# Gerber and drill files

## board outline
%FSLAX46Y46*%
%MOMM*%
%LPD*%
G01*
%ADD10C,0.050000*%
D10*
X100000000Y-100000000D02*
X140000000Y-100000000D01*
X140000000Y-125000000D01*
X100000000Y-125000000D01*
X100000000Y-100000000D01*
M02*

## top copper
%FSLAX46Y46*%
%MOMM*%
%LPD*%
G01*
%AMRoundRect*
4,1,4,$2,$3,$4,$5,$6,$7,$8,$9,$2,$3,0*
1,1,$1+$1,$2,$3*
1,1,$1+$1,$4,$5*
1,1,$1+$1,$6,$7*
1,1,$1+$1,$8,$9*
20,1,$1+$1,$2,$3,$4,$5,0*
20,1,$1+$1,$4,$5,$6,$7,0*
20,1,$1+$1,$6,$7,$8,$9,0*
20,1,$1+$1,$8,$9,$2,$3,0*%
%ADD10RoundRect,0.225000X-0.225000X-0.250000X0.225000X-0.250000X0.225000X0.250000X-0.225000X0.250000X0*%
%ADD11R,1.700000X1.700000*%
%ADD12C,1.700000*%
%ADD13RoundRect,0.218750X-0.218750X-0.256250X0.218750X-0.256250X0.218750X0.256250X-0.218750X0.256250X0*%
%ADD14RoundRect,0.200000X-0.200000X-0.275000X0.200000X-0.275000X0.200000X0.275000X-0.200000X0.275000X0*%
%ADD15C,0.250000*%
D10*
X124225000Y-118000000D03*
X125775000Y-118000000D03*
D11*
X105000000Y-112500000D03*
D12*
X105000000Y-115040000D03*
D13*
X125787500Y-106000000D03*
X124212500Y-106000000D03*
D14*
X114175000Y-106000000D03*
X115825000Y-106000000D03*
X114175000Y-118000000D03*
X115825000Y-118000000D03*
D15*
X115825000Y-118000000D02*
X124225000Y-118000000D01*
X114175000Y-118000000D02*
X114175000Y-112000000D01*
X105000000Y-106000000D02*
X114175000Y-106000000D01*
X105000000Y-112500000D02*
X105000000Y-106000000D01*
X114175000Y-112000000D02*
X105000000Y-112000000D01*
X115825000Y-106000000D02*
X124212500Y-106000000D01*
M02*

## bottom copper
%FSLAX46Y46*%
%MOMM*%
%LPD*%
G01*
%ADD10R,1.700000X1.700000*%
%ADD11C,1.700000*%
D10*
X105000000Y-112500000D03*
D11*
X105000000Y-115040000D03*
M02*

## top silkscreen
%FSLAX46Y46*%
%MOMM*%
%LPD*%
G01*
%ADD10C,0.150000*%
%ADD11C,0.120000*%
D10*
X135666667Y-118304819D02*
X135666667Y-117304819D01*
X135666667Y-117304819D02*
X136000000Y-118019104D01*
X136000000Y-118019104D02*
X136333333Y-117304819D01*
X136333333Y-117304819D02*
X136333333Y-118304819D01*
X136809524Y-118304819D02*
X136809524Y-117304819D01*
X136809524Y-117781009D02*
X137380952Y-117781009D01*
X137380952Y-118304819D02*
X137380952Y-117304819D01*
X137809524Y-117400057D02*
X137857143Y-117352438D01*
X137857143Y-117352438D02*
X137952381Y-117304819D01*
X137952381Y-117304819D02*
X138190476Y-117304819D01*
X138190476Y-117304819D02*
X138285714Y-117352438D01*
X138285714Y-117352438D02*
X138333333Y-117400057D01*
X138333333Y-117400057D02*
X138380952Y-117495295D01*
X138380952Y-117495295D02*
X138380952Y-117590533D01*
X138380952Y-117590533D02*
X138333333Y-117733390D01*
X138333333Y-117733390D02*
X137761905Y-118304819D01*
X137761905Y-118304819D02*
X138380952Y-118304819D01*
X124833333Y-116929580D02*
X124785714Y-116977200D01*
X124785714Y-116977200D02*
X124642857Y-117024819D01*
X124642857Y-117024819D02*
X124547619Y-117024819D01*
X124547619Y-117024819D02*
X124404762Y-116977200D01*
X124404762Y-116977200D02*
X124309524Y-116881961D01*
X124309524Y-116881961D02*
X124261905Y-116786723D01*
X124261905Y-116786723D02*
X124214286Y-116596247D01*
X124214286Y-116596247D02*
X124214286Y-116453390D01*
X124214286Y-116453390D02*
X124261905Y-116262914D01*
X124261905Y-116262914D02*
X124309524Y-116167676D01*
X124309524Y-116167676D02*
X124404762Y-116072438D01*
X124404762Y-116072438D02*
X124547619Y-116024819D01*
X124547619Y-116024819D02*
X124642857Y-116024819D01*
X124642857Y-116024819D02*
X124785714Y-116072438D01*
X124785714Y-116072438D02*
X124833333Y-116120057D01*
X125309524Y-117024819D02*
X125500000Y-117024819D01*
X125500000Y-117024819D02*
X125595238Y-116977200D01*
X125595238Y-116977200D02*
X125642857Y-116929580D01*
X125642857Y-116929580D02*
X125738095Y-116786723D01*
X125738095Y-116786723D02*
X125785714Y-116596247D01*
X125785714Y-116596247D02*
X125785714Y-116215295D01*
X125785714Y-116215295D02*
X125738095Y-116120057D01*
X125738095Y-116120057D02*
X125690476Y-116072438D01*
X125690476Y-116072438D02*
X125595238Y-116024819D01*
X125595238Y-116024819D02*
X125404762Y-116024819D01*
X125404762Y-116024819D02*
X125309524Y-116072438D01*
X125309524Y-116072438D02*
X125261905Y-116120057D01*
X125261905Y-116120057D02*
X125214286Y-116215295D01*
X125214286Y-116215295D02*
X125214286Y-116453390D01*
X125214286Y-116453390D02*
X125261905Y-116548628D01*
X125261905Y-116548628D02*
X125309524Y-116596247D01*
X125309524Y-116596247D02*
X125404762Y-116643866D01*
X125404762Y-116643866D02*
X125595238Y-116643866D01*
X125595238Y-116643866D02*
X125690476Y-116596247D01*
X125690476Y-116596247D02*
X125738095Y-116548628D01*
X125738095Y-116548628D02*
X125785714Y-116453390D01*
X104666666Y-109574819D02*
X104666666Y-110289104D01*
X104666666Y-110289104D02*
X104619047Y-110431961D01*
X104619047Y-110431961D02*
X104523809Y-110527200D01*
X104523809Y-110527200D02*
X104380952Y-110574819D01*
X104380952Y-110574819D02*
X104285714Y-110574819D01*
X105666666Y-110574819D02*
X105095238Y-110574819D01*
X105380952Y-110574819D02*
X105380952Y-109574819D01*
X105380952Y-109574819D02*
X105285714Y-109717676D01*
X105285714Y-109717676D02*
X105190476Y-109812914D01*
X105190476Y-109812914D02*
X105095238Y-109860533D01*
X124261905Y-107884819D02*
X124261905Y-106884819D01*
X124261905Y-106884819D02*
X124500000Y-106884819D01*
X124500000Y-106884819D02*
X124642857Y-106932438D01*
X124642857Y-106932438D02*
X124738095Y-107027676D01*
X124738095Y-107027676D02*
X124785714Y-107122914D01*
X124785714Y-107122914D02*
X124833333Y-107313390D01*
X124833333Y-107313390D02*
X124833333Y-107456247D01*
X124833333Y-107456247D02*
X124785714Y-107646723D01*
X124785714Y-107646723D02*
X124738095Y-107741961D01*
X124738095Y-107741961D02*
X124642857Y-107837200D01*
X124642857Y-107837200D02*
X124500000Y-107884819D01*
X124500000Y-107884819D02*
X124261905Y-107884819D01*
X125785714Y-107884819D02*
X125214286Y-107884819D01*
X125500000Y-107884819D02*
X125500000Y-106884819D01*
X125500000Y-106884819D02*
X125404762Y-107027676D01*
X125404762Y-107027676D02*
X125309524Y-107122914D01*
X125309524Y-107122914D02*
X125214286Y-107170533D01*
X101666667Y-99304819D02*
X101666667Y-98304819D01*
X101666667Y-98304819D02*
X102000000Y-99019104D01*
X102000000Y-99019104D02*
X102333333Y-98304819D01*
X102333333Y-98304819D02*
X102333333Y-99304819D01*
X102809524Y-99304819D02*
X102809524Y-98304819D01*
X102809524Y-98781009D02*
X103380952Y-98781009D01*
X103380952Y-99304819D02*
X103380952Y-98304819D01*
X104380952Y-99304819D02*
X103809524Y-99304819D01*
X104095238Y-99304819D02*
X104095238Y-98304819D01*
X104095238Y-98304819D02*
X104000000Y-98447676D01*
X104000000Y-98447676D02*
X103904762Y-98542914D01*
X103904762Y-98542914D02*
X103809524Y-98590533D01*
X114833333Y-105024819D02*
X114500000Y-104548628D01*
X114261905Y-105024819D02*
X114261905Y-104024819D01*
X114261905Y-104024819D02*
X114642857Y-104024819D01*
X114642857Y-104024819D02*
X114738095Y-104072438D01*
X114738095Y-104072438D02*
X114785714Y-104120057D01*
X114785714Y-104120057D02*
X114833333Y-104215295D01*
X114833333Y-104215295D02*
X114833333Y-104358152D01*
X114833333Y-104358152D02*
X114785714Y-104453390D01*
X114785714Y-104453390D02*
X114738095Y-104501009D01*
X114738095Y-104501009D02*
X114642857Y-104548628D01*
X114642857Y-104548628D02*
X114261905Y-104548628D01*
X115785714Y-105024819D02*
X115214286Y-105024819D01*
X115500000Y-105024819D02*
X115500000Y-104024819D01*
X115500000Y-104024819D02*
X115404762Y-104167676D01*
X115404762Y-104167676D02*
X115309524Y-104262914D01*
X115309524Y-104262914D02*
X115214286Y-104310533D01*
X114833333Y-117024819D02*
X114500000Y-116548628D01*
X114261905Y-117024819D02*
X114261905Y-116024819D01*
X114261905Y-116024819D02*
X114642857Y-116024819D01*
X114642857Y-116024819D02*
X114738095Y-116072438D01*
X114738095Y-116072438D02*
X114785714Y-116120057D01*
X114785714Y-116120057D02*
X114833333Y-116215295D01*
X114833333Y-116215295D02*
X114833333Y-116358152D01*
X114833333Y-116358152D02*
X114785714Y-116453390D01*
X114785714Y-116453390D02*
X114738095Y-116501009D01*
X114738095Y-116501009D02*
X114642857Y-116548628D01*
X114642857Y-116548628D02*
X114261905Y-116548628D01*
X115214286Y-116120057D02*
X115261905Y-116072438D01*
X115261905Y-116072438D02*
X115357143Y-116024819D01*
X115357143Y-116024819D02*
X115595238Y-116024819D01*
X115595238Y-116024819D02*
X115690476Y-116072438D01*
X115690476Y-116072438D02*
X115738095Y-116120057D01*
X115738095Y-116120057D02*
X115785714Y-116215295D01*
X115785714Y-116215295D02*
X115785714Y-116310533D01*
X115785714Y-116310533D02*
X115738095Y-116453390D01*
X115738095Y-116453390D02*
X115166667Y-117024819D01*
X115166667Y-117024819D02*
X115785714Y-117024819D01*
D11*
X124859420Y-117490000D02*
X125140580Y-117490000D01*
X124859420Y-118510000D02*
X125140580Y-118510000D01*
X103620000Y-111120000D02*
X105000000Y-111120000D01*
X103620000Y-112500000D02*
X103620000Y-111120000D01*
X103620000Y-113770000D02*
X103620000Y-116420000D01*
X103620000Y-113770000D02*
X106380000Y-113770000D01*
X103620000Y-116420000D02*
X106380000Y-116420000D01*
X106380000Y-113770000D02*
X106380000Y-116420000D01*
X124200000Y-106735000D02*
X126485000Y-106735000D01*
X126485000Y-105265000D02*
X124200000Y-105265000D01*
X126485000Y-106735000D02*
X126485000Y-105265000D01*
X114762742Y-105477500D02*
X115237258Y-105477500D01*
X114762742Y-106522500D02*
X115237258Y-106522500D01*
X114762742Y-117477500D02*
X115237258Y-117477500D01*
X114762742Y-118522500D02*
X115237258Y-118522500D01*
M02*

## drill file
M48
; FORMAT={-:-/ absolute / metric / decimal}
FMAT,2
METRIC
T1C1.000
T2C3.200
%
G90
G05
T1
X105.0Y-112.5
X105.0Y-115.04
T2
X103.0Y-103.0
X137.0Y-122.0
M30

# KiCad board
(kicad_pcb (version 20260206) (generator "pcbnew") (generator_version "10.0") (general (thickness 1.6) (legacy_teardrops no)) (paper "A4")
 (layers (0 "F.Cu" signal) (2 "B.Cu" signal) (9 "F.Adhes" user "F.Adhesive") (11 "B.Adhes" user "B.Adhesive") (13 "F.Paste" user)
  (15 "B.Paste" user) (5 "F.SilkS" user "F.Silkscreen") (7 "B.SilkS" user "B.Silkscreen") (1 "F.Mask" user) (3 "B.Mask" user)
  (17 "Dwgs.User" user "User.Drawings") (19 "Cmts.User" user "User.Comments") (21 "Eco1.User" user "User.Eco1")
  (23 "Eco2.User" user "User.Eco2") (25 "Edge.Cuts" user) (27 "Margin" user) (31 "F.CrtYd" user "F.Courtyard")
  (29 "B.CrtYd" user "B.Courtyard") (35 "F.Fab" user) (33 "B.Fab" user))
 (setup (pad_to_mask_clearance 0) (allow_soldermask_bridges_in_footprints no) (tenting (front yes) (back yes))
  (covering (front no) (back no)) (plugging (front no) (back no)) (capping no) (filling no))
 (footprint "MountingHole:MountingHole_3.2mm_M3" (layer "F.Cu") (at 137 122)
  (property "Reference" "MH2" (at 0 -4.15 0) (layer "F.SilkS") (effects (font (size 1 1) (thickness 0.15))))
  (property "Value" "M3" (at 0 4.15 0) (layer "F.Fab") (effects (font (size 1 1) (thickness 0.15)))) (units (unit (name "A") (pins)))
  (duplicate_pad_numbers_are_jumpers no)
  (pad "" np_thru_hole circle (at 0 0) (size 3.2 3.2) (drill 3.2) (layers "*.Cu" "*.Mask")))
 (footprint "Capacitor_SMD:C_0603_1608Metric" (layer "F.Cu") (at 125 118)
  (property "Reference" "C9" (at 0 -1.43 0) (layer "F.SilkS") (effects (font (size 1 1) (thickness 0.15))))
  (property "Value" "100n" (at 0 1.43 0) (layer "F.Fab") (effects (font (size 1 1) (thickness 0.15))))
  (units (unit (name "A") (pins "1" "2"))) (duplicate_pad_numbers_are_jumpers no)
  (fp_line (start -0.14058 -0.51) (end 0.14058 -0.51) (stroke (width 0.12) (type solid)) (layer "F.SilkS"))
  (fp_line (start -0.14058 0.51) (end 0.14058 0.51) (stroke (width 0.12) (type solid)) (layer "F.SilkS"))
  (pad "1" smd roundrect (at -0.775 0) (size 0.9 0.95) (layers "F.Cu" "F.Mask" "F.Paste") (roundrect_rratio 0.25) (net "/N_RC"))
  (pad "2" smd roundrect (at 0.775 0) (size 0.9 0.95) (layers "F.Cu" "F.Mask" "F.Paste") (roundrect_rratio 0.25) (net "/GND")))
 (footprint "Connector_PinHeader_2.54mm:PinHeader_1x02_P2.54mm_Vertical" (layer "F.Cu") (at 105 112.5)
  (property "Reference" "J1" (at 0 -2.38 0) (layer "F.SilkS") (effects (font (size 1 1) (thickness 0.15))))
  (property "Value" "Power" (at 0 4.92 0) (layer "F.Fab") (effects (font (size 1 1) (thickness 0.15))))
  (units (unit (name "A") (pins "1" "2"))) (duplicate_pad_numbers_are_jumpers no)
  (fp_line (start -1.38 -1.38) (end 0 -1.38) (stroke (width 0.12) (type solid)) (layer "F.SilkS"))
  (fp_line (start -1.38 0) (end -1.38 -1.38) (stroke (width 0.12) (type solid)) (layer "F.SilkS"))
  (fp_line (start -1.38 1.27) (end -1.38 3.92) (stroke (width 0.12) (type solid)) (layer "F.SilkS"))
  (fp_line (start -1.38 1.27) (end 1.38 1.27) (stroke (width 0.12) (type solid)) (layer "F.SilkS"))
  (fp_line (start -1.38 3.92) (end 1.38 3.92) (stroke (width 0.12) (type solid)) (layer "F.SilkS"))
  (fp_line (start 1.38 1.27) (end 1.38 3.92) (stroke (width 0.12) (type solid)) (layer "F.SilkS"))
  (pad "1" thru_hole rect (at 0 0) (size 1.7 1.7) (drill 1) (layers "*.Cu" "*.Mask") (remove_unused_layers no) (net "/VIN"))
  (pad "2" thru_hole circle (at 0 2.54) (size 1.7 1.7) (drill 1) (layers "*.Cu" "*.Mask") (remove_unused_layers no) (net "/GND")))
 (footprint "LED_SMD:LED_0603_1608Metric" (layer "F.Cu") (at 125 106 180)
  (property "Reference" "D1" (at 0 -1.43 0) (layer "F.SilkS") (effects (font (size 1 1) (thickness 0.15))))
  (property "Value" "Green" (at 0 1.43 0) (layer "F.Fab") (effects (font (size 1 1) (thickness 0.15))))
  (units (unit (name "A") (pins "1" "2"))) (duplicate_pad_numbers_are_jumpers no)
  (fp_line (start 0.8 -0.735) (end -1.485 -0.735) (stroke (width 0.12) (type solid)) (layer "F.SilkS"))
  (fp_line (start -1.485 0.735) (end 0.8 0.735) (stroke (width 0.12) (type solid)) (layer "F.SilkS"))
  (fp_line (start -1.485 -0.735) (end -1.485 0.735) (stroke (width 0.12) (type solid)) (layer "F.SilkS"))
  (pad "1" smd roundrect (at -0.7875 0) (size 0.875 0.95) (layers "F.Cu" "F.Mask" "F.Paste") (roundrect_rratio 0.25) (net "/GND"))
  (pad "2" smd roundrect (at 0.7875 0) (size 0.875 0.95) (layers "F.Cu" "F.Mask" "F.Paste") (roundrect_rratio 0.25) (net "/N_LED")))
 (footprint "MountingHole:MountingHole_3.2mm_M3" (layer "F.Cu") (at 103 103)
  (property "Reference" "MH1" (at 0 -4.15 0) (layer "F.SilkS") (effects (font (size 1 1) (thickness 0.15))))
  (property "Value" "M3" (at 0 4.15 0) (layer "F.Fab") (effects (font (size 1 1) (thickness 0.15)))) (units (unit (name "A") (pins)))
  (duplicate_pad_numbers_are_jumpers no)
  (pad "" np_thru_hole circle (at 0 0) (size 3.2 3.2) (drill 3.2) (layers "*.Cu" "*.Mask")))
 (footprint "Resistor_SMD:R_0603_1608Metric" (layer "F.Cu") (at 115 106)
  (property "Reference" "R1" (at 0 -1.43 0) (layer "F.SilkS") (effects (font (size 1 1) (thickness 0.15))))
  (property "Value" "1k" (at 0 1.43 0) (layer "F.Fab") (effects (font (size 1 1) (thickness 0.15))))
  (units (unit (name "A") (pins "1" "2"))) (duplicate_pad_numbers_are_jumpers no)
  (fp_line (start -0.237258 -0.5225) (end 0.237258 -0.5225) (stroke (width 0.12) (type solid)) (layer "F.SilkS"))
  (fp_line (start -0.237258 0.5225) (end 0.237258 0.5225) (stroke (width 0.12) (type solid)) (layer "F.SilkS"))
  (pad "1" smd roundrect (at -0.825 0) (size 0.8 0.95) (layers "F.Cu" "F.Mask" "F.Paste") (roundrect_rratio 0.25) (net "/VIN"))
  (pad "2" smd roundrect (at 0.825 0) (size 0.8 0.95) (layers "F.Cu" "F.Mask" "F.Paste") (roundrect_rratio 0.25) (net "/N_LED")))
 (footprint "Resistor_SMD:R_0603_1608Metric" (layer "F.Cu") (at 115 118)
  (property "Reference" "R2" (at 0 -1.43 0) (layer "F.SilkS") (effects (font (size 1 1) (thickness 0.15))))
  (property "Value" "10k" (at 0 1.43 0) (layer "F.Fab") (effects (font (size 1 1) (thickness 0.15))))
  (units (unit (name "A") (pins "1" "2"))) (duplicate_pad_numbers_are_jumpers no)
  (fp_line (start -0.237258 -0.5225) (end 0.237258 -0.5225) (stroke (width 0.12) (type solid)) (layer "F.SilkS"))
  (fp_line (start -0.237258 0.5225) (end 0.237258 0.5225) (stroke (width 0.12) (type solid)) (layer "F.SilkS"))
  (pad "1" smd roundrect (at -0.825 0) (size 0.8 0.95) (layers "F.Cu" "F.Mask" "F.Paste") (roundrect_rratio 0.25) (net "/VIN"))
  (pad "2" smd roundrect (at 0.825 0) (size 0.8 0.95) (layers "F.Cu" "F.Mask" "F.Paste") (roundrect_rratio 0.25) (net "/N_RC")))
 (gr_rect (start 100 100) (end 140 125) (stroke (width 0.05) (type default)) (fill no) (layer "Edge.Cuts"))
 (segment (start 115.825 118) (end 124.225 118) (width 0.25) (layer "F.Cu") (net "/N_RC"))
 (segment (start 114.175 118) (end 114.175 112) (width 0.25) (layer "F.Cu") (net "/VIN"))
 (segment (start 105 106) (end 114.175 106) (width 0.25) (layer "F.Cu") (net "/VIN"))
 (segment (start 105 112.5) (end 105 106) (width 0.25) (layer "F.Cu") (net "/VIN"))
 (segment (start 114.175 112) (end 105 112) (width 0.25) (layer "F.Cu") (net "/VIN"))
 (segment (start 115.825 106) (end 124.2125 106) (width 0.25) (layer "F.Cu") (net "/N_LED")))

